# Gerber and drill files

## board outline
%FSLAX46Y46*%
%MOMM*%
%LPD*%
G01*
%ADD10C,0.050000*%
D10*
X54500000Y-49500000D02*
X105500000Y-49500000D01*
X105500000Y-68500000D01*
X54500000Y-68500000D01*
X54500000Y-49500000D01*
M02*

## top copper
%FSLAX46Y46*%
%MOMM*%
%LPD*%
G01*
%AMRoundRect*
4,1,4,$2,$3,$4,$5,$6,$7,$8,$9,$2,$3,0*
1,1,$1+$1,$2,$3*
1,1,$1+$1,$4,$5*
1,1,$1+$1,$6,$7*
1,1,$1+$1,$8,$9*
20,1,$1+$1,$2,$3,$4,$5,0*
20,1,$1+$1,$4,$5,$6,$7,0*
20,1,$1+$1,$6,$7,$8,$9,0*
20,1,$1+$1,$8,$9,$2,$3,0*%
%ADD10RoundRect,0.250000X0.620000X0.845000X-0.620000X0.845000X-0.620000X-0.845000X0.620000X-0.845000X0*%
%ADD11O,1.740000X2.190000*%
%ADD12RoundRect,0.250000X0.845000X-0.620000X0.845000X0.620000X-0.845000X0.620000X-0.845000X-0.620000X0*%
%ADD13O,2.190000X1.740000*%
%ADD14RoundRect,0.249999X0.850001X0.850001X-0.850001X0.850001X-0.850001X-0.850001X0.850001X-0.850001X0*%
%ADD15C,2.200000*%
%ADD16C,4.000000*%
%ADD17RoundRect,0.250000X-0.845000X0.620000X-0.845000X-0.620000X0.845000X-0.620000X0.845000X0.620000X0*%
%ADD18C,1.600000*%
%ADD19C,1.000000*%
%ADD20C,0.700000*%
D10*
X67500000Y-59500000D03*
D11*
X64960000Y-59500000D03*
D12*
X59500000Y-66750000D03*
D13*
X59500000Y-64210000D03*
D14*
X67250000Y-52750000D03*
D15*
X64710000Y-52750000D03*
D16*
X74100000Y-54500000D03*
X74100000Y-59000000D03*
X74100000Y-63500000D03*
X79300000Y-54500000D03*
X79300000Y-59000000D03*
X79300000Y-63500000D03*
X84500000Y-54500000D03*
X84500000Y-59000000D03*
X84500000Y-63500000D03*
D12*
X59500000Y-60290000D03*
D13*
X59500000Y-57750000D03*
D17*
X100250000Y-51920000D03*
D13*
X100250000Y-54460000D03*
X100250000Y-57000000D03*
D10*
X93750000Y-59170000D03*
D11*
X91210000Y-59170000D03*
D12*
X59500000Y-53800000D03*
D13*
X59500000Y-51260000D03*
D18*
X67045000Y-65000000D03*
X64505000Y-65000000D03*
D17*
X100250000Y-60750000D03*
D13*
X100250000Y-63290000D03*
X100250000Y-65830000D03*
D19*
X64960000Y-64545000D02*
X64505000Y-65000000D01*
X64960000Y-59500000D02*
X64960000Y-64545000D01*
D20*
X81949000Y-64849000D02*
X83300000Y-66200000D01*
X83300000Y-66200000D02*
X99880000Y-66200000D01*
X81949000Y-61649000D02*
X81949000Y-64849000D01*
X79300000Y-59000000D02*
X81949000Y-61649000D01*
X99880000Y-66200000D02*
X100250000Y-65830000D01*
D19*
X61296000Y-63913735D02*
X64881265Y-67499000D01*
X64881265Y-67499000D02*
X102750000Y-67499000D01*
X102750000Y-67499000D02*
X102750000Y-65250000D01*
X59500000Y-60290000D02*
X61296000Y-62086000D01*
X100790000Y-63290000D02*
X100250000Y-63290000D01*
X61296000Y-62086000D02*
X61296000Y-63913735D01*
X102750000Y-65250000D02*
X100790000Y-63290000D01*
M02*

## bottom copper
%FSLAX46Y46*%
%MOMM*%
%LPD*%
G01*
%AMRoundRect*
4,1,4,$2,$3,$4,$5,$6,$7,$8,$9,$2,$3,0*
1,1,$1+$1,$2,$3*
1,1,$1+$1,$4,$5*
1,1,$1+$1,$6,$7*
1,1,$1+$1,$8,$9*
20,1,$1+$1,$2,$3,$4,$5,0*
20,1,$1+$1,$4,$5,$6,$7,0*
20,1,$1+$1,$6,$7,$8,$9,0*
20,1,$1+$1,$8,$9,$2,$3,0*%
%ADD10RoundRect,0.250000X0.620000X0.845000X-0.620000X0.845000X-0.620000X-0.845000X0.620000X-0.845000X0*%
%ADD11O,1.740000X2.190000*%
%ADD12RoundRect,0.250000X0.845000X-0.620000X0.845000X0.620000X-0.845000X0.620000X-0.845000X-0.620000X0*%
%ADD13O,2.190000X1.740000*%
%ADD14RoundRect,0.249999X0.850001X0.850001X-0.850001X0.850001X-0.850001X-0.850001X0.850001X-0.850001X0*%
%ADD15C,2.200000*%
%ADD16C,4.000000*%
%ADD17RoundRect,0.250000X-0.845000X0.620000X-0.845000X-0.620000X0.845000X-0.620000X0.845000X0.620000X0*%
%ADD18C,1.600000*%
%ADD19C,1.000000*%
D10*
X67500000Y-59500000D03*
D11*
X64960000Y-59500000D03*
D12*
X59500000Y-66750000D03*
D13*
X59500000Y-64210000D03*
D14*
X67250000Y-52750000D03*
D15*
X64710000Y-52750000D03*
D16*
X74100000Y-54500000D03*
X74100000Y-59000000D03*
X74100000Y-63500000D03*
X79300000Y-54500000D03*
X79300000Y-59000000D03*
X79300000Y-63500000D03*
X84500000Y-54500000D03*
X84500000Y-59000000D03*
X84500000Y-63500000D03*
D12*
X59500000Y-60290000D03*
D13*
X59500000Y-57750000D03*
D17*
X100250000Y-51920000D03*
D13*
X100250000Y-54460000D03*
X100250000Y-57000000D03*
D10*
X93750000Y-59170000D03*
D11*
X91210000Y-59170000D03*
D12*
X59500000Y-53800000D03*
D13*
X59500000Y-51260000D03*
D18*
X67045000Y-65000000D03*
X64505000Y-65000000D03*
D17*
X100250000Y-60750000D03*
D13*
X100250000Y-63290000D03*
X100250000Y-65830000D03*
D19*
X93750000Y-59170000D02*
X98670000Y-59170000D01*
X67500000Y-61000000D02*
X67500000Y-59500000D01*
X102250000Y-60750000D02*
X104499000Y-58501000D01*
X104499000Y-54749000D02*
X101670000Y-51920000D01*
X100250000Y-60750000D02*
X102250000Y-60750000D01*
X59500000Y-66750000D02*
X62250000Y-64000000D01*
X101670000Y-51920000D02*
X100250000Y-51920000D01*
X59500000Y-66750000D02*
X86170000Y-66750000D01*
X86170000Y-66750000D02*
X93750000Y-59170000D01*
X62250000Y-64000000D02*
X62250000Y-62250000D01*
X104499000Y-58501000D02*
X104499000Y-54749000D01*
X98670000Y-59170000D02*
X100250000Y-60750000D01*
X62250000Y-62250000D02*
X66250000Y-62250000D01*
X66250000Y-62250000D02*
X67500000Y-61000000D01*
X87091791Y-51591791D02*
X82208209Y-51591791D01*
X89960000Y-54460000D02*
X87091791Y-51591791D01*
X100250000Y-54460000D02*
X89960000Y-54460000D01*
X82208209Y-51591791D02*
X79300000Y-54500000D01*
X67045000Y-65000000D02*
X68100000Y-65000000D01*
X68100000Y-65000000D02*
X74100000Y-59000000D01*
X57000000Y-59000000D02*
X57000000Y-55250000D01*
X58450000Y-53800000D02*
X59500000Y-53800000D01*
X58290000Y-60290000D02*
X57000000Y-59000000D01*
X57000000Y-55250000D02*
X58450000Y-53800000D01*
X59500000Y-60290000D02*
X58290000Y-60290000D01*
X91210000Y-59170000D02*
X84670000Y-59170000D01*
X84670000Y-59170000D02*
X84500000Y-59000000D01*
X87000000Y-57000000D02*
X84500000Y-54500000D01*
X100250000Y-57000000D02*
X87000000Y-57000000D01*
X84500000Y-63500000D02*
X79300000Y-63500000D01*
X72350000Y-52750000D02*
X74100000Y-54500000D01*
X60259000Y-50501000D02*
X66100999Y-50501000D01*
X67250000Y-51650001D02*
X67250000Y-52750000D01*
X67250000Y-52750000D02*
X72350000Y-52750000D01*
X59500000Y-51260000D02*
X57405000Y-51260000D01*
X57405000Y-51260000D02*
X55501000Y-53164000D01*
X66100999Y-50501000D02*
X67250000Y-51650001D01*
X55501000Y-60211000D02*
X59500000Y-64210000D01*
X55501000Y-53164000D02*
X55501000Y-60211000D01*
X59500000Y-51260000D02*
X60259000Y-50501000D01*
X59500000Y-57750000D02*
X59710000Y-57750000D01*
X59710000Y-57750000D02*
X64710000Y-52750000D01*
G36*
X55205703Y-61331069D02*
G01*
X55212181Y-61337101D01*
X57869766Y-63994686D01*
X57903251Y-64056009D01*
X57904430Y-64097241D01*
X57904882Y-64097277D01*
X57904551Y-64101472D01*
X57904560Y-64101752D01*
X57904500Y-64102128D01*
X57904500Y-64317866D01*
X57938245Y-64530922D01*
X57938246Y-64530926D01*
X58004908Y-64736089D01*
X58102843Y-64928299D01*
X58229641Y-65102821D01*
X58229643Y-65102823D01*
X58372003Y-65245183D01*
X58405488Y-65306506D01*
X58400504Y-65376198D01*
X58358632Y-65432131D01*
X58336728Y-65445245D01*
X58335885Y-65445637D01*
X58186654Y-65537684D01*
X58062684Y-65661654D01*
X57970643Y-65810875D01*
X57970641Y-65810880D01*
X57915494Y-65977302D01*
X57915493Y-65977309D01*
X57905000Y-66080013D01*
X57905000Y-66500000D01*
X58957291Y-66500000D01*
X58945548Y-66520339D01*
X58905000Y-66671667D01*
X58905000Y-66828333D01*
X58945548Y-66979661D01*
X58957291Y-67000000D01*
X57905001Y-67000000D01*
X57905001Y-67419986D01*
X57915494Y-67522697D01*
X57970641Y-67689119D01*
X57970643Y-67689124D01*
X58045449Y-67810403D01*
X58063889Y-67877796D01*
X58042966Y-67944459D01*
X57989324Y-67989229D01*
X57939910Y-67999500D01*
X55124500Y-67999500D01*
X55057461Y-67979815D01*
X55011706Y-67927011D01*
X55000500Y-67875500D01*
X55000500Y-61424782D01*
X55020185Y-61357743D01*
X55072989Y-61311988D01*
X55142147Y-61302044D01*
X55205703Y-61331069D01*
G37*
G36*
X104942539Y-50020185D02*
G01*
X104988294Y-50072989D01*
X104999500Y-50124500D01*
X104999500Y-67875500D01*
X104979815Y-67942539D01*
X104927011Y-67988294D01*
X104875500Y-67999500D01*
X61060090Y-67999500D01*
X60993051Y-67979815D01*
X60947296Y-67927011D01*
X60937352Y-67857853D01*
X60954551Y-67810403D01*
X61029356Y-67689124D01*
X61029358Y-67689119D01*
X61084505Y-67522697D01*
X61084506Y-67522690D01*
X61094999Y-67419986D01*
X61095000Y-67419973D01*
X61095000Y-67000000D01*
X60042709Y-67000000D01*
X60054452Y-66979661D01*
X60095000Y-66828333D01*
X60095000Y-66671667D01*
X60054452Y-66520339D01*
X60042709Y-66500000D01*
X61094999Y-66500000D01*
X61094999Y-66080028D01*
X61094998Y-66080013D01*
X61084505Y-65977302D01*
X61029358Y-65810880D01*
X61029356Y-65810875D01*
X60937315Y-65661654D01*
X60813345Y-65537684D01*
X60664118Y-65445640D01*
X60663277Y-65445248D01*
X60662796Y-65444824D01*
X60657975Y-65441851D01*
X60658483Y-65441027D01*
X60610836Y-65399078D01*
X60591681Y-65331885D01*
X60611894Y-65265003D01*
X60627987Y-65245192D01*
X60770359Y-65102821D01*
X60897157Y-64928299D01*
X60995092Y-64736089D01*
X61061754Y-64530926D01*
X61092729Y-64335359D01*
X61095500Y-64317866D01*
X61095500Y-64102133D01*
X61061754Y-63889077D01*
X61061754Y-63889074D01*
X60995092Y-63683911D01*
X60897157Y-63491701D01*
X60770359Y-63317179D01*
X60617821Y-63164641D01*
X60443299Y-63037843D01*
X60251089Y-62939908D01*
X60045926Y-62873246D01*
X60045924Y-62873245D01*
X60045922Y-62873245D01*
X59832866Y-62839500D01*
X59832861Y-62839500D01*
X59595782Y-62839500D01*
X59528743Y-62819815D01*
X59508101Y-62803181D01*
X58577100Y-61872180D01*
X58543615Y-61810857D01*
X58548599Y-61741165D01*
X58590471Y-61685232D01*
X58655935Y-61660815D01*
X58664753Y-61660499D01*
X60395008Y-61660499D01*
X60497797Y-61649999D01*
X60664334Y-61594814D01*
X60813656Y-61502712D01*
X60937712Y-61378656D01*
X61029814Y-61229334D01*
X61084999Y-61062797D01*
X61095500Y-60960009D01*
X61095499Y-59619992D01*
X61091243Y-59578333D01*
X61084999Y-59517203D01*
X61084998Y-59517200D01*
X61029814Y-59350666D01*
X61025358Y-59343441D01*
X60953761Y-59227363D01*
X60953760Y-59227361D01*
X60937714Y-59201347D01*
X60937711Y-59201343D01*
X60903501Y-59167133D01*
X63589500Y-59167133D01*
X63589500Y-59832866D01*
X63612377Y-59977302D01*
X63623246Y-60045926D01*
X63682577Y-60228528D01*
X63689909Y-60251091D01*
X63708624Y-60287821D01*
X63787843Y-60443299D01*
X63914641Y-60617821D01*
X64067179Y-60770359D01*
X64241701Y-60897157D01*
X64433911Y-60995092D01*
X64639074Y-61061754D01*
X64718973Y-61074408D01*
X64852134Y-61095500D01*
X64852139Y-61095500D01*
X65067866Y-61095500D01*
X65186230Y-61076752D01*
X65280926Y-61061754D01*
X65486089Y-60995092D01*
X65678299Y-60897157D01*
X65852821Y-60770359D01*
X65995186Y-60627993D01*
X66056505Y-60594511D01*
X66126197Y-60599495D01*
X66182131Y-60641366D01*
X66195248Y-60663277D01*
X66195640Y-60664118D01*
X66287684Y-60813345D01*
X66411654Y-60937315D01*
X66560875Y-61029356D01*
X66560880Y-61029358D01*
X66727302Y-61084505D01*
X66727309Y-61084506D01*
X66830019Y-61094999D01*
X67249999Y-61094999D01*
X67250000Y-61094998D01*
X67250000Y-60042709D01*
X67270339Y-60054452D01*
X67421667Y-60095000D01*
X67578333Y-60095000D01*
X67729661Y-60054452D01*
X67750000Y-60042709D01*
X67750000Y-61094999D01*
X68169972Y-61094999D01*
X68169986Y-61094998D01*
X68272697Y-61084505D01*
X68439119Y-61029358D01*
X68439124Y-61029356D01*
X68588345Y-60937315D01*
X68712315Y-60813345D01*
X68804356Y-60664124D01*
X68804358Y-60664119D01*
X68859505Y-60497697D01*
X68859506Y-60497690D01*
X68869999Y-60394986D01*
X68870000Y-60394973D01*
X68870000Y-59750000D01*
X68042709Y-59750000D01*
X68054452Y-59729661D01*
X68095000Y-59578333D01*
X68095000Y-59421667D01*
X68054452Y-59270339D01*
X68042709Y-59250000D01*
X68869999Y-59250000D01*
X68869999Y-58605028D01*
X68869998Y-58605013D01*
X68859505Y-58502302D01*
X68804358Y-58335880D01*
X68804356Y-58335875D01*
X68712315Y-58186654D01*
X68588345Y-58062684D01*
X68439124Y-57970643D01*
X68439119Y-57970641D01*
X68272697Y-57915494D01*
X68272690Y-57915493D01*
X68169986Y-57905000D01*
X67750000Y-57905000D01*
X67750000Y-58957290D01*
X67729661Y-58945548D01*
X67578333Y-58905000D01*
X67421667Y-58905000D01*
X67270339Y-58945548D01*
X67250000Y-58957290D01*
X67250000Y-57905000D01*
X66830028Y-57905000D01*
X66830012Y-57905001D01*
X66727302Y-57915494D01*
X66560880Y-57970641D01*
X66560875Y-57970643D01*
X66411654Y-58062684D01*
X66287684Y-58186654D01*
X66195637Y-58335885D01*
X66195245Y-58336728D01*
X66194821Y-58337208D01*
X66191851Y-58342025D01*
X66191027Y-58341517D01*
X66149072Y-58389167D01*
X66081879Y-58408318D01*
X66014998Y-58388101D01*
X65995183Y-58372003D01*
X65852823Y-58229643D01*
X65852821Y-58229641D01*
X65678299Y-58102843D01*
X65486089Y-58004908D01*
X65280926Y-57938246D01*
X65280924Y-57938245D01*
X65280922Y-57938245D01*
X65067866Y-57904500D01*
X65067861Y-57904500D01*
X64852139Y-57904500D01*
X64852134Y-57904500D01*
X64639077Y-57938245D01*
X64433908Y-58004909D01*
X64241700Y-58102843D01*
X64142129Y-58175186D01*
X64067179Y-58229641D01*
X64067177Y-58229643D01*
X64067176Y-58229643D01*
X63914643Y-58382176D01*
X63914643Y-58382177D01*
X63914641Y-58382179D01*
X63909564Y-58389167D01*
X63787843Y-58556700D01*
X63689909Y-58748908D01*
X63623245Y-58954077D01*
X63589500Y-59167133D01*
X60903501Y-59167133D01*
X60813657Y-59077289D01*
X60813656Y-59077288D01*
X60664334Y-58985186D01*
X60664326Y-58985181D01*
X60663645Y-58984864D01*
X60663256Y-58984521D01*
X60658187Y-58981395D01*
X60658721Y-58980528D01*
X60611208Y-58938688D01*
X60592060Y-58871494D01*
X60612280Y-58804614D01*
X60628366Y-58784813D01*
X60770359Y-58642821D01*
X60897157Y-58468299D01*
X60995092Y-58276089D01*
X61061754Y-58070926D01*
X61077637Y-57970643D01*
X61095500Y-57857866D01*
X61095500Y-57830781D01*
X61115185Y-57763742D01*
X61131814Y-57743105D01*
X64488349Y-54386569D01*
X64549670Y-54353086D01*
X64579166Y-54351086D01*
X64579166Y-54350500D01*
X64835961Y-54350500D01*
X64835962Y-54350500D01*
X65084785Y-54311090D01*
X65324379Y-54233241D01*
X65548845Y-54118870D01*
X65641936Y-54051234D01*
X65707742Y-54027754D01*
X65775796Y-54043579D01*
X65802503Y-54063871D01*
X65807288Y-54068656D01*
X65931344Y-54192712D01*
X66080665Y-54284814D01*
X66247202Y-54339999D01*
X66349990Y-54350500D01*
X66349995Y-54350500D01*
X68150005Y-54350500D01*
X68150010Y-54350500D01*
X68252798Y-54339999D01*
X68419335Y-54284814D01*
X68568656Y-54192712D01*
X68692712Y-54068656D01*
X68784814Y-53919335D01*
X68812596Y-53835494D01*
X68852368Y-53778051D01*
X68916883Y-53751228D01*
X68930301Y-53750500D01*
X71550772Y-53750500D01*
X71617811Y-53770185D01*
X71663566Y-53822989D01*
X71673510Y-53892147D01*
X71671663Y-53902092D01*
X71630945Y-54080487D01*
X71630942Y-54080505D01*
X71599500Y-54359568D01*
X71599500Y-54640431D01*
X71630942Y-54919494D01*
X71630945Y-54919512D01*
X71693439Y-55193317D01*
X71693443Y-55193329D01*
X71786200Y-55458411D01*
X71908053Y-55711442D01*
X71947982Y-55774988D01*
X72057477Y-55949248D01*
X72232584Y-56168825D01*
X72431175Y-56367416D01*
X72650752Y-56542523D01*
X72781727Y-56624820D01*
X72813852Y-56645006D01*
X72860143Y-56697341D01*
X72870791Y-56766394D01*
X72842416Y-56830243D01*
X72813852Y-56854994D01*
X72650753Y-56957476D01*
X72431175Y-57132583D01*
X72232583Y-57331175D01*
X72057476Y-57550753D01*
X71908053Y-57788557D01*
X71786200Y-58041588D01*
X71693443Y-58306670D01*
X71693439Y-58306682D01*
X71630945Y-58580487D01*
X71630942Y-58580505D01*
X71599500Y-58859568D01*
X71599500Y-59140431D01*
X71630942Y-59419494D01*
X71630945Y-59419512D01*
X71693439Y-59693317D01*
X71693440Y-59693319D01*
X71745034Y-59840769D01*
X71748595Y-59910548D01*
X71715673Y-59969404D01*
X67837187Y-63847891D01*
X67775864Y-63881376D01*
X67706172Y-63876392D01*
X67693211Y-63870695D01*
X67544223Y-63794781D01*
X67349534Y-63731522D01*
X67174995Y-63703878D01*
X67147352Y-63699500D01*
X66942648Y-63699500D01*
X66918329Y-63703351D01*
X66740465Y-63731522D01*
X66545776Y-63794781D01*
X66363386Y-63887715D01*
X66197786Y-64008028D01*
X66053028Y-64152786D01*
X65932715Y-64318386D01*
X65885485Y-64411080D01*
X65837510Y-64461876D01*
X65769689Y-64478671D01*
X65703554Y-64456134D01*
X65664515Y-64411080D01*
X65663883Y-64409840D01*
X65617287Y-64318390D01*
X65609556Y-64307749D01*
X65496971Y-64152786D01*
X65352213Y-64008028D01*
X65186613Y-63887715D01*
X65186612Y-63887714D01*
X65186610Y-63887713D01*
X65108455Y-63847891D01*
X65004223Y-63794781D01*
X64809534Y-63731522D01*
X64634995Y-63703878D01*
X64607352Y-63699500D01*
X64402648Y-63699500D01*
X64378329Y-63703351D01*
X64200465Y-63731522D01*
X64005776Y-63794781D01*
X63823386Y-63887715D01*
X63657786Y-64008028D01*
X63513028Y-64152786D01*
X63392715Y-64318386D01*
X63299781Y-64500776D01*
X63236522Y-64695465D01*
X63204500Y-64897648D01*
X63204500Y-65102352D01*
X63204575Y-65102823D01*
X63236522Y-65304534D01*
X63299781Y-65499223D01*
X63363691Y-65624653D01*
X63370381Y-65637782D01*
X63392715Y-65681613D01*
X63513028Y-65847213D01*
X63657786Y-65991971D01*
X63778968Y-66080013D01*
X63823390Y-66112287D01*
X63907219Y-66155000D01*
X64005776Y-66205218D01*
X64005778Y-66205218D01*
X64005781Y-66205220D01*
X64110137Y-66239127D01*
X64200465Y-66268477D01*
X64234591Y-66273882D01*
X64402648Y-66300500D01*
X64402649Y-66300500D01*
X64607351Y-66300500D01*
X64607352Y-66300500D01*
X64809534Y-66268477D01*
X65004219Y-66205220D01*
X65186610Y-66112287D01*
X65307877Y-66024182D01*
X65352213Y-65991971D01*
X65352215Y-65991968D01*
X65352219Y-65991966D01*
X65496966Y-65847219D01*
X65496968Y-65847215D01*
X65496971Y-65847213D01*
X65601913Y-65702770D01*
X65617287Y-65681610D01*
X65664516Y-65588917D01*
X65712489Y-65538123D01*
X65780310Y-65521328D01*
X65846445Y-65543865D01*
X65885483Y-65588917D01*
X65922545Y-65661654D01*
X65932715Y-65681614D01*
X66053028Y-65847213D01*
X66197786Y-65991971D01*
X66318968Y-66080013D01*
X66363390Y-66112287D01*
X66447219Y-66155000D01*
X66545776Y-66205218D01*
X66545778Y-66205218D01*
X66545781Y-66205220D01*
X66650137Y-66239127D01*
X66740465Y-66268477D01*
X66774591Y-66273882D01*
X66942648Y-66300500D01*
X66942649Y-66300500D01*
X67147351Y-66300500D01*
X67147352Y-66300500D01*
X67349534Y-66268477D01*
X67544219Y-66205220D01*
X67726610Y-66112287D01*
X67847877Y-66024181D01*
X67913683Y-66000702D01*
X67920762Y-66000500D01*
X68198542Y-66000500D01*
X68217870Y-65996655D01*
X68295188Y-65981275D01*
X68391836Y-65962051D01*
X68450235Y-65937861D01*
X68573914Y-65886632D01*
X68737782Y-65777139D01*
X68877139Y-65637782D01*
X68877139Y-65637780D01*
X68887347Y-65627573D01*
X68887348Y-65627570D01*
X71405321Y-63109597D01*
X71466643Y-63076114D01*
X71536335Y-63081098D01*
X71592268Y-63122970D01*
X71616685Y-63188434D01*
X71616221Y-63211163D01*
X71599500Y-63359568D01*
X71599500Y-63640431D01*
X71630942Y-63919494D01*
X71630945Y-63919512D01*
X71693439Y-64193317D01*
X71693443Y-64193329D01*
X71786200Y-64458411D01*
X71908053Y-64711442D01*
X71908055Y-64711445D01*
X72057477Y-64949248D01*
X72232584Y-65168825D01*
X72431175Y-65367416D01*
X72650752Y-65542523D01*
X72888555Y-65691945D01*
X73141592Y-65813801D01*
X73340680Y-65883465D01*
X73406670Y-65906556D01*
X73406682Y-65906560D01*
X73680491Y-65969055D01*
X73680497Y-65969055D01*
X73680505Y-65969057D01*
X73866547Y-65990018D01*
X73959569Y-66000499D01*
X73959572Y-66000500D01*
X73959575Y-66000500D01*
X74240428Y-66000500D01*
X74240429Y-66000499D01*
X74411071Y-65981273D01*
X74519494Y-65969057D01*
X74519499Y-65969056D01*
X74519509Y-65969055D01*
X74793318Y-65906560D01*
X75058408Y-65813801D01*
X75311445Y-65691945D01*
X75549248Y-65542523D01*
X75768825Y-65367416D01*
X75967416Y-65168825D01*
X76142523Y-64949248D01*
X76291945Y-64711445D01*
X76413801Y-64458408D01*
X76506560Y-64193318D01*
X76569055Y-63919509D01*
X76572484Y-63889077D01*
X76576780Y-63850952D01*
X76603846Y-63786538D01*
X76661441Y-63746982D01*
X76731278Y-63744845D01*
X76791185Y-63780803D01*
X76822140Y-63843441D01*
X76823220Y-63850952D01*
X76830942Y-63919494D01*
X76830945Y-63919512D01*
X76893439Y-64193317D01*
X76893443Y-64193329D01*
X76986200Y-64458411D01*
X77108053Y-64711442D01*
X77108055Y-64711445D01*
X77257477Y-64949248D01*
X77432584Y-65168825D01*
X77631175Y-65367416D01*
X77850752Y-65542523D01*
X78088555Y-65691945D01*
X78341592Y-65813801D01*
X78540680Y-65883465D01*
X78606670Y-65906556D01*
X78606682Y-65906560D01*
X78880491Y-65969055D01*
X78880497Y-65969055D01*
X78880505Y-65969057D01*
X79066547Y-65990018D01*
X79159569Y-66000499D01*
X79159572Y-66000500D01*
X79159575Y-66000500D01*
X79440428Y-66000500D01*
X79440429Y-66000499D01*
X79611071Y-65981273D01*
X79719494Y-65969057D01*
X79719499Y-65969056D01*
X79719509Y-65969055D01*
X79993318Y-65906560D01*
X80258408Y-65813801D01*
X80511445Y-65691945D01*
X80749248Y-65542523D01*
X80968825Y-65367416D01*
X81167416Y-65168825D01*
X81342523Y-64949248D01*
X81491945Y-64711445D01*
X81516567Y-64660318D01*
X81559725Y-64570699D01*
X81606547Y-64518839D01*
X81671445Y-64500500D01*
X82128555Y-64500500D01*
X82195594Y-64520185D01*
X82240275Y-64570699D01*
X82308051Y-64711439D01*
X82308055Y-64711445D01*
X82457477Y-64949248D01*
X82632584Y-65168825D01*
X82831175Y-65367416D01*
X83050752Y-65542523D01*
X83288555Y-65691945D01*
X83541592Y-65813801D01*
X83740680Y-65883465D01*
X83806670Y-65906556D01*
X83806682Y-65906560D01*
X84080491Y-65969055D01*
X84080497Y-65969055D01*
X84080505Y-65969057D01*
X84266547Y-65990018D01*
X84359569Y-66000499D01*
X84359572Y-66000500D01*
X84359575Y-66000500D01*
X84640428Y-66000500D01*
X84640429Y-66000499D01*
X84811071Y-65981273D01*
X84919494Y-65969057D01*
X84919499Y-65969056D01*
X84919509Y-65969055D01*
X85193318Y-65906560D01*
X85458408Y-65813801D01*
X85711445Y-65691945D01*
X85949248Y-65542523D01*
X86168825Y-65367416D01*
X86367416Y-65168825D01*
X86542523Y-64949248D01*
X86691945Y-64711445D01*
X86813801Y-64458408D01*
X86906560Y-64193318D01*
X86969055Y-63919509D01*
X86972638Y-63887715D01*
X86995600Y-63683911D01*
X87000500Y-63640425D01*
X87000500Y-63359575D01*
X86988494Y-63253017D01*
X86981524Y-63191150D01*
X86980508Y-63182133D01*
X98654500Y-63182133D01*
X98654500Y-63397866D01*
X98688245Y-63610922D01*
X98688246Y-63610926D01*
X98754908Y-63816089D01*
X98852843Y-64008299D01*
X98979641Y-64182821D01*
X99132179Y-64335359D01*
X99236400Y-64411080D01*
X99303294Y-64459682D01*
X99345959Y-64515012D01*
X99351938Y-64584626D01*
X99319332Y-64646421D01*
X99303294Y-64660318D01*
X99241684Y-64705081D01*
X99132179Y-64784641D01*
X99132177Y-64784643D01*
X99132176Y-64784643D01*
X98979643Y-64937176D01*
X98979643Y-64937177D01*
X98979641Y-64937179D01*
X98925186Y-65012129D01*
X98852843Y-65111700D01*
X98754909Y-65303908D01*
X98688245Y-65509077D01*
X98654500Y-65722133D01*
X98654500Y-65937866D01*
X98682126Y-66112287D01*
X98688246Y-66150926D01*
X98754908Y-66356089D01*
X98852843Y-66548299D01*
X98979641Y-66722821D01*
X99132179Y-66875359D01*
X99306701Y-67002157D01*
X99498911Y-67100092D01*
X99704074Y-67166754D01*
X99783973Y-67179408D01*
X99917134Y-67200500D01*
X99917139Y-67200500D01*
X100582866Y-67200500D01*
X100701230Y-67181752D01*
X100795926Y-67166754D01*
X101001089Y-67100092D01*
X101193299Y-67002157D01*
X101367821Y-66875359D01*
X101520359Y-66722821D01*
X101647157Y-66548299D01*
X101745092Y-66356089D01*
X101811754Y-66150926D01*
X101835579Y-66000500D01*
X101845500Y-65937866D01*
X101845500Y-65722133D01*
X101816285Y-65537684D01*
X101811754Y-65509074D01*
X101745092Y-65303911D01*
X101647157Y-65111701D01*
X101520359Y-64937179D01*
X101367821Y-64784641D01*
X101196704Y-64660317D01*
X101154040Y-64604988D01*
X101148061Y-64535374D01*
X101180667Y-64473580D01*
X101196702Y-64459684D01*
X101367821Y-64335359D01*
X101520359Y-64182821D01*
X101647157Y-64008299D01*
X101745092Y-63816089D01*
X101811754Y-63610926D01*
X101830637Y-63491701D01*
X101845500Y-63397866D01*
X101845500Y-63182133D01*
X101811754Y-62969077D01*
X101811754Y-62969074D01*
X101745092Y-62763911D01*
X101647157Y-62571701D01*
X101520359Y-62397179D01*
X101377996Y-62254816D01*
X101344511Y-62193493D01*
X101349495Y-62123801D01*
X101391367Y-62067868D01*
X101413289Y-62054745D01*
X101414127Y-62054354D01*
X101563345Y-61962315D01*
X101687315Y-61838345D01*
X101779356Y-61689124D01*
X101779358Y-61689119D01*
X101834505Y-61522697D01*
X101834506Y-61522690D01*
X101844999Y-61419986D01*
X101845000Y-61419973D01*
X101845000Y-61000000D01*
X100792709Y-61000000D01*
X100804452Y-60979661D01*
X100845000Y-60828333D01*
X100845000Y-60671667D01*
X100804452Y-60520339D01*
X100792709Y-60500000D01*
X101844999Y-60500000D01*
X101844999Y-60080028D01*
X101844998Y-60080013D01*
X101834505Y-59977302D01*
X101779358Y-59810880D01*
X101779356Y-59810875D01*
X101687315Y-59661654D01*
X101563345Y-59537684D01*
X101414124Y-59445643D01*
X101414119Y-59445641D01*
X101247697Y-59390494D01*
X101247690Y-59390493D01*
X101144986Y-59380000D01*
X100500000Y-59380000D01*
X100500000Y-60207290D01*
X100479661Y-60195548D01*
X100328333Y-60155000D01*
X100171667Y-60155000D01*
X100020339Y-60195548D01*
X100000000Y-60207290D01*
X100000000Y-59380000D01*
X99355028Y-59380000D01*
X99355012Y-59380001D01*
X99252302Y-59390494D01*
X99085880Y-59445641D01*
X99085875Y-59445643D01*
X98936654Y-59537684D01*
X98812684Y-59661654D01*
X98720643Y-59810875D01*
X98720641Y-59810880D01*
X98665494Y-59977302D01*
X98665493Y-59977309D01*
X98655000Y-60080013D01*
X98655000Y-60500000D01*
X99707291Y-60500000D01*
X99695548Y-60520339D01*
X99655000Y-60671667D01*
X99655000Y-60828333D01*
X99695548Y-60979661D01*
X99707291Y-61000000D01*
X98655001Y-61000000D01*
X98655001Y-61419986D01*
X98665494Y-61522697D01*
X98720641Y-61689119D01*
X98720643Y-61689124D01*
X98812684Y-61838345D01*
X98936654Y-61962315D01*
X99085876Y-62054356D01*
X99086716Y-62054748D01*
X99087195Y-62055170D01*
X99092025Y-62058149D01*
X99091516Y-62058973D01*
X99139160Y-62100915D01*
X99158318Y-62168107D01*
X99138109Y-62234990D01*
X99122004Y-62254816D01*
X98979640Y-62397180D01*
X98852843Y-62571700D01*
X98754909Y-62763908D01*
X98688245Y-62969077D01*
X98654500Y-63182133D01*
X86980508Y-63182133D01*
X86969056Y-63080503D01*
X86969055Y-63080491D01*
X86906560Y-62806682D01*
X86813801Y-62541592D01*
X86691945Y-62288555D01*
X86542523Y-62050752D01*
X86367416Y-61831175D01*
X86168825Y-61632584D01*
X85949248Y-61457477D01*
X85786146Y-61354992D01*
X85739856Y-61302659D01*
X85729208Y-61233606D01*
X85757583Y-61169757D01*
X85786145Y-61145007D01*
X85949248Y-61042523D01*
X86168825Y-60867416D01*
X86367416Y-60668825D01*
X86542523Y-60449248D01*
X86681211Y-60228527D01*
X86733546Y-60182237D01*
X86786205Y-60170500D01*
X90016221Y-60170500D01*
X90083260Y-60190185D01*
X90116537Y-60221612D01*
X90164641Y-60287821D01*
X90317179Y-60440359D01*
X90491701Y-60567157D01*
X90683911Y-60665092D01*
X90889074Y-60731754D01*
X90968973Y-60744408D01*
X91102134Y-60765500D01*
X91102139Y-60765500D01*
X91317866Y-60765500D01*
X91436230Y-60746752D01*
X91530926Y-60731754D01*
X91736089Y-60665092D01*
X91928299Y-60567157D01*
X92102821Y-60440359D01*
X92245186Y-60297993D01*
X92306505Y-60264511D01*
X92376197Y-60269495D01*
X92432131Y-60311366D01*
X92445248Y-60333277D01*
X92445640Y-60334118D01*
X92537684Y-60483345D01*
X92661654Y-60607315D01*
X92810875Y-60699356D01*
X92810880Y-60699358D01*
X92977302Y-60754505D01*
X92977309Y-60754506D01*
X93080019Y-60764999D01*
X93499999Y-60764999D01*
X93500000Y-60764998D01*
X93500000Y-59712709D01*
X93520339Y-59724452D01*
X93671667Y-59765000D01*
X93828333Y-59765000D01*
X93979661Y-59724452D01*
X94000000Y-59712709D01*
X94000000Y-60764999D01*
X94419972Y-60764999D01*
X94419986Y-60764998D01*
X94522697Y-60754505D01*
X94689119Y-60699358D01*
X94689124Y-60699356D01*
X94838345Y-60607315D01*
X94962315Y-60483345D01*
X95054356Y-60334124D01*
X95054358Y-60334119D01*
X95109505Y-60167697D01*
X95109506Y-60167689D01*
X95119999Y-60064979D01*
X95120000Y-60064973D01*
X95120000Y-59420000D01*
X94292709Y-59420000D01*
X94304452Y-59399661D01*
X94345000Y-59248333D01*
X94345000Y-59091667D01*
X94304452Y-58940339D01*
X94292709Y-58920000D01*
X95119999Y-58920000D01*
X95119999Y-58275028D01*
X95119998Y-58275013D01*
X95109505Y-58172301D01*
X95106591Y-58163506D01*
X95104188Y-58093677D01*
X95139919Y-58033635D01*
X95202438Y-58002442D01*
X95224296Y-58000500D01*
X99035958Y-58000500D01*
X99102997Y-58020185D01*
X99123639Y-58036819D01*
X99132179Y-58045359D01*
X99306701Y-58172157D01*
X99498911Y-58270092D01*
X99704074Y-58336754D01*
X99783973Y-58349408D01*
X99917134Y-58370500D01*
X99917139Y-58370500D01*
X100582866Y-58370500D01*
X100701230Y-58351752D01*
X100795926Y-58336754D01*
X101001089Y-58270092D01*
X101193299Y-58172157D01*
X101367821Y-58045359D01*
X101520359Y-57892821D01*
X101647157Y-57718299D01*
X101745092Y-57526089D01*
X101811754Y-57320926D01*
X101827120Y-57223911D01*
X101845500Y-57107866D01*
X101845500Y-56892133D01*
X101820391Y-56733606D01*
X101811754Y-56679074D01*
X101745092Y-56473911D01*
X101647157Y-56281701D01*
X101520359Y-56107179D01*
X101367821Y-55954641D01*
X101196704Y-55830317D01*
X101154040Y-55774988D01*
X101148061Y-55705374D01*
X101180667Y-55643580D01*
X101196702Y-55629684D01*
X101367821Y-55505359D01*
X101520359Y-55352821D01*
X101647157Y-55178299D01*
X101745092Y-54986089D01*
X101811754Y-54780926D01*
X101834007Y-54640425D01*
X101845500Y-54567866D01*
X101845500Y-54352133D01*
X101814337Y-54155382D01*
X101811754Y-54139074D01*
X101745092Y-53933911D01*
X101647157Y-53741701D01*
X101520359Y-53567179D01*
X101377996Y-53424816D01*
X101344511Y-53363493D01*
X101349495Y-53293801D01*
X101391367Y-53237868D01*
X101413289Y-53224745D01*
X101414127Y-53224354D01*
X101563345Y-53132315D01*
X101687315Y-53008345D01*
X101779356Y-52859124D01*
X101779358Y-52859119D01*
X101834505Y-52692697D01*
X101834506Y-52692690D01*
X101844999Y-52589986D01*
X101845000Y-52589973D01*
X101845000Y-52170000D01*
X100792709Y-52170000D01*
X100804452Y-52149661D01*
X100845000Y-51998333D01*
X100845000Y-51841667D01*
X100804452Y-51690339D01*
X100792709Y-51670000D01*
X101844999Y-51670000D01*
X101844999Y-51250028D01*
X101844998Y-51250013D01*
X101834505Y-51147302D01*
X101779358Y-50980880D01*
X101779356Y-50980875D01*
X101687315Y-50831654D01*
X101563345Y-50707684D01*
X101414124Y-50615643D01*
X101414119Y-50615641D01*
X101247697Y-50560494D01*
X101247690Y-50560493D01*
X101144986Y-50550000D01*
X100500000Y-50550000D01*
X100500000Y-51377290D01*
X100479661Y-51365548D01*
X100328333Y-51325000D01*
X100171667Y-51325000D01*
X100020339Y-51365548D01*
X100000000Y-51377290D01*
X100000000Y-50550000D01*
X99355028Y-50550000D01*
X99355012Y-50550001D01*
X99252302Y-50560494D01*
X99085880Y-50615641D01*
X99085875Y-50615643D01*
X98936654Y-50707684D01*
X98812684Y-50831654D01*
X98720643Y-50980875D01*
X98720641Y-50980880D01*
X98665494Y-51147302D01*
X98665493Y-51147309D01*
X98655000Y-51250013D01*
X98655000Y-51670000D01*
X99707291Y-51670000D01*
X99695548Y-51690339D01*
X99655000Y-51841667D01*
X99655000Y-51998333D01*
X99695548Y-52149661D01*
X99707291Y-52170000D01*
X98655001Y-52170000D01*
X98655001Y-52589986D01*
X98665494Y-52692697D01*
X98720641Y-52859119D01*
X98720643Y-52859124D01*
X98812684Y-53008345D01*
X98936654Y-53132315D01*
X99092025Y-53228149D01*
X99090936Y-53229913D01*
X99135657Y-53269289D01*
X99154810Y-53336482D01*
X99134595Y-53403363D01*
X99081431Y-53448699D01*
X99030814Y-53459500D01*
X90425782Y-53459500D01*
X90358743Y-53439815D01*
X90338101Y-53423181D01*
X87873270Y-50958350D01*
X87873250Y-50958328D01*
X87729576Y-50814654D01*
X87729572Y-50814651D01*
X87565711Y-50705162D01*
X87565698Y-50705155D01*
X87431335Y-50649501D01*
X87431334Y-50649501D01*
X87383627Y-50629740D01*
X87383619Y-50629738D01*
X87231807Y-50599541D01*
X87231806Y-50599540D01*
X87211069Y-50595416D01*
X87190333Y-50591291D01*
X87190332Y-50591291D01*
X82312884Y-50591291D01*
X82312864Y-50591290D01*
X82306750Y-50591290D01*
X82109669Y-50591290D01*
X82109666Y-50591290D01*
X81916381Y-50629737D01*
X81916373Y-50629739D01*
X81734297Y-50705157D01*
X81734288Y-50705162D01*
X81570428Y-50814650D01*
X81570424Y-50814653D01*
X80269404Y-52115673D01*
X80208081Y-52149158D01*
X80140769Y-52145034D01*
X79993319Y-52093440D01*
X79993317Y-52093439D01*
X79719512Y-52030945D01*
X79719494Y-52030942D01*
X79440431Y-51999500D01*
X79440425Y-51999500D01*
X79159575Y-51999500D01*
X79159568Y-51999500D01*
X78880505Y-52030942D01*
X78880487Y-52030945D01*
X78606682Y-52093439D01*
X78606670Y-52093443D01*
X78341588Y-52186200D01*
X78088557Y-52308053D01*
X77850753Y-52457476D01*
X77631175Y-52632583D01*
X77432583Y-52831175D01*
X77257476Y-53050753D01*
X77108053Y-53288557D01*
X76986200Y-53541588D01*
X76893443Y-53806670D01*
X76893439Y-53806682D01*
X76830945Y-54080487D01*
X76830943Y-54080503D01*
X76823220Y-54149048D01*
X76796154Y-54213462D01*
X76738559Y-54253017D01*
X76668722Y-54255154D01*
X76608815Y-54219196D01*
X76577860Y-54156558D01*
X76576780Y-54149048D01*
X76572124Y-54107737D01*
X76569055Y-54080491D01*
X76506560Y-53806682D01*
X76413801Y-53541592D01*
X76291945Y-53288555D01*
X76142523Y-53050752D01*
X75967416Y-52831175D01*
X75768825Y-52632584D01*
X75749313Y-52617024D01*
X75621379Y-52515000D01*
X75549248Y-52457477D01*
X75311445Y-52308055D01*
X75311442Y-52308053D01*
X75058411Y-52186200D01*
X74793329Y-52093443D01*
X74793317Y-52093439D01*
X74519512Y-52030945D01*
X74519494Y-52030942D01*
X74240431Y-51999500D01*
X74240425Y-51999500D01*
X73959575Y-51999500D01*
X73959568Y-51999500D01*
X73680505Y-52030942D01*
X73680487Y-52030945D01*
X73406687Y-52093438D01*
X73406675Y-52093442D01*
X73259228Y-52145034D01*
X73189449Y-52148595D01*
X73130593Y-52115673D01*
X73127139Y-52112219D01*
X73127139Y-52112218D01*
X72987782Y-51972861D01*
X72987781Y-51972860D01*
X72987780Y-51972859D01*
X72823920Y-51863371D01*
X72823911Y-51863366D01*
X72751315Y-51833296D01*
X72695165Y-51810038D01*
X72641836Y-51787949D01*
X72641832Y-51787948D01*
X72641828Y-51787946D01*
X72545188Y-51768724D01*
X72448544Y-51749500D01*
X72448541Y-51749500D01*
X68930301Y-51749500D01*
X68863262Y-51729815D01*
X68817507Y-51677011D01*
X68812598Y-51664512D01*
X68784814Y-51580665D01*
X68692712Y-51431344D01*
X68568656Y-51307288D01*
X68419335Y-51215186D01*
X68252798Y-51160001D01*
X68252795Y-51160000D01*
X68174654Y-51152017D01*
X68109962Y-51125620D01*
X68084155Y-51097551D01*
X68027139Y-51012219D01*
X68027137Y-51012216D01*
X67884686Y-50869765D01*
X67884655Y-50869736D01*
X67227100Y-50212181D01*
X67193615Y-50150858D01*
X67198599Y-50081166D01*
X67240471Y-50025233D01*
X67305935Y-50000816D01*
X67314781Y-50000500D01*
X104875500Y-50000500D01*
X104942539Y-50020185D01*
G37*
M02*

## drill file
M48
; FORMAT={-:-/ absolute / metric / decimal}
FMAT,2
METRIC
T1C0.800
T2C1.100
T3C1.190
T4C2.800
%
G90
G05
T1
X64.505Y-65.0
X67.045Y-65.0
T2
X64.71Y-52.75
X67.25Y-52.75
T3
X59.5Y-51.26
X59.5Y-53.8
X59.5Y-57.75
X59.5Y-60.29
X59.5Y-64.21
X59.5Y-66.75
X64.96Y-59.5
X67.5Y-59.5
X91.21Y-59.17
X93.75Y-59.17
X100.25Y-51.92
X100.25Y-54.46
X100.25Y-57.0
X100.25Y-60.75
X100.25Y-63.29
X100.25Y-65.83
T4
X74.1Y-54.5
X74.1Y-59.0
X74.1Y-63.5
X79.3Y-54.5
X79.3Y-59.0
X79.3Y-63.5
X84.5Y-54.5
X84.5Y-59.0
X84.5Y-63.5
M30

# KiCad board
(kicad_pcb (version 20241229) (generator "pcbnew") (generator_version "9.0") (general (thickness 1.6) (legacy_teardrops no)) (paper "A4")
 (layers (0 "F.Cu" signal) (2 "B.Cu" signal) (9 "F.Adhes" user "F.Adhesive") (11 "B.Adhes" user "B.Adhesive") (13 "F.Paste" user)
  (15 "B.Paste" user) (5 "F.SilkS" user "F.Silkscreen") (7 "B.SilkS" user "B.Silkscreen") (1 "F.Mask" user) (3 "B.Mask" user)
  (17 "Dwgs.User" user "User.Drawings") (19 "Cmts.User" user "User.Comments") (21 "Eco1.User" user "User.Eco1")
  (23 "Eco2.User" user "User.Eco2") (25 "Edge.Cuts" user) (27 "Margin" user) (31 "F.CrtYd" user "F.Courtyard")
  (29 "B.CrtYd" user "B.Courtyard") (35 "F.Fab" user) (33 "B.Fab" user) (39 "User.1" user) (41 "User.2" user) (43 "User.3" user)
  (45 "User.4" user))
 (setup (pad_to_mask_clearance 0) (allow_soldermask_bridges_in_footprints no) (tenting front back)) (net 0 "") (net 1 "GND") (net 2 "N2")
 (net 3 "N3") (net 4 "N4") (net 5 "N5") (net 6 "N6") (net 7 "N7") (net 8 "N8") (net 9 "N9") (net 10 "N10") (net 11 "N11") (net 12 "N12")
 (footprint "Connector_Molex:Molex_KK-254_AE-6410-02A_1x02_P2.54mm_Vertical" (layer "F.Cu") (at 67.5 59.5 180)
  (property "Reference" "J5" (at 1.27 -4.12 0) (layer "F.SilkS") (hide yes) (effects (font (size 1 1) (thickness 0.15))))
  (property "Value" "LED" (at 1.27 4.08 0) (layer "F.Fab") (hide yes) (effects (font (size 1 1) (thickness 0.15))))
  (pad "1" thru_hole roundrect (at 0 0 180) (size 1.74 2.19) (drill 1.19) (layers "*.Cu" "*.Mask") (remove_unused_layers no)
   (roundrect_rratio 0.143678) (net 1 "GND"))
  (pad "2" thru_hole oval (at 2.54 0 180) (size 1.74 2.19) (drill 1.19) (layers "*.Cu" "*.Mask") (remove_unused_layers no) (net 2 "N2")))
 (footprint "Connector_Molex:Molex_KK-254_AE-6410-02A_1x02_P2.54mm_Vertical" (layer "F.Cu") (at 59.5 66.75 90)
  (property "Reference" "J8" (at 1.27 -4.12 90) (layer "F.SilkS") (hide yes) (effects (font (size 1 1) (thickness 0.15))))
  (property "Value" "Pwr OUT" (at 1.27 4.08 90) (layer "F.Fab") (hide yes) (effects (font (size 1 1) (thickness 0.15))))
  (pad "1" thru_hole roundrect (at 0 0 90) (size 1.74 2.19) (drill 1.19) (layers "*.Cu" "*.Mask") (remove_unused_layers no)
   (roundrect_rratio 0.143678) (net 1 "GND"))
  (pad "2" thru_hole oval (at 2.54 0 90) (size 1.74 2.19) (drill 1.19) (layers "*.Cu" "*.Mask") (remove_unused_layers no) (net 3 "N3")))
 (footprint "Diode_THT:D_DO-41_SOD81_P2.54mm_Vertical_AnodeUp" (layer "F.Cu") (at 67.25 52.75 180)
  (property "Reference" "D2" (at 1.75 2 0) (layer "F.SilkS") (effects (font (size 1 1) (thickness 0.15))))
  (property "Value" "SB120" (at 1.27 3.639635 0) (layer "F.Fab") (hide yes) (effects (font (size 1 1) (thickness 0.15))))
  (pad "1" thru_hole roundrect (at 0 0 180) (size 2.2 2.2) (drill 1.1) (layers "*.Cu" "*.Mask") (remove_unused_layers no)
   (roundrect_rratio 0.113636) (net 3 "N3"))
  (pad "2" thru_hole circle (at 2.54 0 180) (size 2.2 2.2) (drill 1.1) (layers "*.Cu" "*.Mask") (remove_unused_layers no) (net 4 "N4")))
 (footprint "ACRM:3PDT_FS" (layer "F.Cu") (at 77.1 58)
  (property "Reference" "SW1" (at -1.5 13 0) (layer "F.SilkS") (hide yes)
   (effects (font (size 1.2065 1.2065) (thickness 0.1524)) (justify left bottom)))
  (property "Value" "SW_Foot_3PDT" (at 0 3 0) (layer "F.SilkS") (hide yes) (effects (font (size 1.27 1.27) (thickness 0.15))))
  (pad "A1" thru_hole circle (at -3 -3.5 180) (size 4 4) (drill 2.8) (layers "*.Cu" "*.Mask") (remove_unused_layers no) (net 3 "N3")
   (solder_mask_margin 0.1016))
  (pad "A2" thru_hole circle (at -3 1 180) (size 4 4) (drill 2.8) (layers "*.Cu" "*.Mask") (remove_unused_layers no) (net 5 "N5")
   (solder_mask_margin 0.1016))
  (pad "A3" thru_hole circle (at -3 5.5 180) (size 4 4) (drill 2.8) (layers "*.Cu" "*.Mask") (remove_unused_layers no) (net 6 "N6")
   (solder_mask_margin 0.1016))
  (pad "B1" thru_hole circle (at 2.2 -3.5 180) (size 4 4) (drill 2.8) (layers "*.Cu" "*.Mask") (remove_unused_layers no) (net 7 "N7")
   (solder_mask_margin 0.1016))
  (pad "B2" thru_hole circle (at 2.2 1 180) (size 4 4) (drill 2.8) (layers "*.Cu" "*.Mask") (remove_unused_layers no) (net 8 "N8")
   (solder_mask_margin 0.1016))
  (pad "B3" thru_hole circle (at 2.2 5.5 180) (size 4 4) (drill 2.8) (layers "*.Cu" "*.Mask") (remove_unused_layers no) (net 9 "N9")
   (solder_mask_margin 0.1016))
  (pad "C1" thru_hole circle (at 7.4 -3.5 180) (size 4 4) (drill 2.8) (layers "*.Cu" "*.Mask") (remove_unused_layers no) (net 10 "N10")
   (solder_mask_margin 0.1016))
  (pad "C2" thru_hole circle (at 7.4 1 180) (size 4 4) (drill 2.8) (layers "*.Cu" "*.Mask") (remove_unused_layers no) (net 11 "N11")
   (solder_mask_margin 0.1016))
  (pad "C3" thru_hole circle (at 7.4 5.5 180) (size 4 4) (drill 2.8) (layers "*.Cu" "*.Mask") (remove_unused_layers no) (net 9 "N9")
   (solder_mask_margin 0.1016)))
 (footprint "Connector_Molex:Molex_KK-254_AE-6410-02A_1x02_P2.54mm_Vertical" (layer "F.Cu") (at 59.5 60.29 90)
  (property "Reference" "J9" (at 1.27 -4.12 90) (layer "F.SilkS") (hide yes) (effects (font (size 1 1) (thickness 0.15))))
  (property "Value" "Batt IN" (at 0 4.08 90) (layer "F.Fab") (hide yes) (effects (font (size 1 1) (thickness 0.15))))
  (pad "1" thru_hole roundrect (at 0 0 90) (size 1.74 2.19) (drill 1.19) (layers "*.Cu" "*.Mask") (remove_unused_layers no)
   (roundrect_rratio 0.143678) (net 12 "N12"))
  (pad "2" thru_hole oval (at 2.54 0 90) (size 1.74 2.19) (drill 1.19) (layers "*.Cu" "*.Mask") (remove_unused_layers no) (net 4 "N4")))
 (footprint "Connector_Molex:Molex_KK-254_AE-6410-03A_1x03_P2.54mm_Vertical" (layer "F.Cu") (at 100.25 51.92 -90)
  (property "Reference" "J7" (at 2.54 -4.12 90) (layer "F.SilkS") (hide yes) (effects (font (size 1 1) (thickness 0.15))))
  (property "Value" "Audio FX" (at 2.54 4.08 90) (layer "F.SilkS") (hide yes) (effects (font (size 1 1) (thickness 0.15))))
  (pad "1" thru_hole roundrect (at 0 0 270) (size 1.74 2.19) (drill 1.19) (layers "*.Cu" "*.Mask") (remove_unused_layers no)
   (roundrect_rratio 0.143678) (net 1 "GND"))
  (pad "2" thru_hole oval (at 2.54 0 270) (size 1.74 2.19) (drill 1.19) (layers "*.Cu" "*.Mask") (remove_unused_layers no) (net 7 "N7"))
  (pad "3" thru_hole oval (at 5.08 0 270) (size 1.74 2.19) (drill 1.19) (layers "*.Cu" "*.Mask") (remove_unused_layers no) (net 10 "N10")))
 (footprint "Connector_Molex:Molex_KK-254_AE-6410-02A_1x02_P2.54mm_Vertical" (layer "F.Cu") (at 93.75 59.17 180)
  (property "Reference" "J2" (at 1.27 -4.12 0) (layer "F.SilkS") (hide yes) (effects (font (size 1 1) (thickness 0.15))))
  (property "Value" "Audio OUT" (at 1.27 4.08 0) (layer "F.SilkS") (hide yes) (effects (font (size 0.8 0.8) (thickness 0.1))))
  (pad "1" thru_hole roundrect (at 0 0 180) (size 1.74 2.19) (drill 1.19) (layers "*.Cu" "*.Mask") (remove_unused_layers no)
   (roundrect_rratio 0.143678) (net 1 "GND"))
  (pad "2" thru_hole oval (at 2.54 0 180) (size 1.74 2.19) (drill 1.19) (layers "*.Cu" "*.Mask") (remove_unused_layers no) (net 11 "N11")))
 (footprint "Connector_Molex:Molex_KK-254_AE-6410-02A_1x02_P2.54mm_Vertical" (layer "F.Cu") (at 59.5 53.8 90)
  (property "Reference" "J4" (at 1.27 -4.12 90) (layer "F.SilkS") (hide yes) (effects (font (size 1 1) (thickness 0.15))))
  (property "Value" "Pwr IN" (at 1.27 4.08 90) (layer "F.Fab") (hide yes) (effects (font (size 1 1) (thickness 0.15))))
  (pad "1" thru_hole roundrect (at 0 0 90) (size 1.74 2.19) (drill 1.19) (layers "*.Cu" "*.Mask") (remove_unused_layers no)
   (roundrect_rratio 0.143678) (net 12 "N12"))
  (pad "2" thru_hole oval (at 2.54 0 90) (size 1.74 2.19) (drill 1.19) (layers "*.Cu" "*.Mask") (remove_unused_layers no) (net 3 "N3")))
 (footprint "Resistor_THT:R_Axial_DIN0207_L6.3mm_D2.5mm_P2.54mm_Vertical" (layer "F.Cu") (at 67.045 65 180)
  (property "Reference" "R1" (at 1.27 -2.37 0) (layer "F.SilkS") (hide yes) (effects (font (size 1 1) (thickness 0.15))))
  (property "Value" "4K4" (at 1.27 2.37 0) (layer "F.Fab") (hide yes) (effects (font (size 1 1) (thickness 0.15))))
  (pad "1" thru_hole circle (at 0 0 180) (size 1.6 1.6) (drill 0.8) (layers "*.Cu" "*.Mask") (remove_unused_layers no) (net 5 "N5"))
  (pad "2" thru_hole circle (at 2.54 0 180) (size 1.6 1.6) (drill 0.8) (layers "*.Cu" "*.Mask") (remove_unused_layers no) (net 2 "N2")))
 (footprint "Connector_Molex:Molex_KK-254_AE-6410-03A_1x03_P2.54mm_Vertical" (layer "F.Cu") (at 100.25 60.75 -90)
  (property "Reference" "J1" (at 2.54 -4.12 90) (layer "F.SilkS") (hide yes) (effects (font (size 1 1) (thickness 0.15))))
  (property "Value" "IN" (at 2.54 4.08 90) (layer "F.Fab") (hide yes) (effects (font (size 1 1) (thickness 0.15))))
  (pad "1" thru_hole roundrect (at 0 0 270) (size 1.74 2.19) (drill 1.19) (layers "*.Cu" "*.Mask") (remove_unused_layers no)
   (roundrect_rratio 0.143678) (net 1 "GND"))
  (pad "2" thru_hole oval (at 2.54 0 270) (size 1.74 2.19) (drill 1.19) (layers "*.Cu" "*.Mask") (remove_unused_layers no) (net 12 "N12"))
  (pad "3" thru_hole oval (at 5.08 0 270) (size 1.74 2.19) (drill 1.19) (layers "*.Cu" "*.Mask") (remove_unused_layers no) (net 8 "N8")))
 (gr_rect (start 54.5 49.5) (end 105.5 68.5) (stroke (width 0.05) (type default)) (fill no) (layer "Edge.Cuts"))
 (segment (start 93.75 59.17) (end 98.67 59.17) (width 1) (layer "B.Cu") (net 1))
 (segment (start 67.5 61) (end 67.5 59.5) (width 1) (layer "B.Cu") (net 1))
 (segment (start 102.25 60.75) (end 104.499 58.501) (width 1) (layer "B.Cu") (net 1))
 (segment (start 104.499 54.749) (end 101.67 51.92) (width 1) (layer "B.Cu") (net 1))
 (segment (start 100.25 60.75) (end 102.25 60.75) (width 1) (layer "B.Cu") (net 1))
 (segment (start 59.5 66.75) (end 62.25 64) (width 1) (layer "B.Cu") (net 1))
 (segment (start 101.67 51.92) (end 100.25 51.92) (width 1) (layer "B.Cu") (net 1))
 (segment (start 59.5 66.75) (end 86.17 66.75) (width 1) (layer "B.Cu") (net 1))
 (segment (start 86.17 66.75) (end 93.75 59.17) (width 1) (layer "B.Cu") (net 1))
 (segment (start 62.25 64) (end 62.25 62.25) (width 1) (layer "B.Cu") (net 1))
 (segment (start 104.499 58.501) (end 104.499 54.749) (width 1) (layer "B.Cu") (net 1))
 (segment (start 98.67 59.17) (end 100.25 60.75) (width 1) (layer "B.Cu") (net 1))
 (segment (start 62.25 62.25) (end 66.25 62.25) (width 1) (layer "B.Cu") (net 1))
 (segment (start 66.25 62.25) (end 67.5 61) (width 1) (layer "B.Cu") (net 1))
 (segment (start 64.96 64.545) (end 64.505 65) (width 1) (layer "F.Cu") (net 2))
 (segment (start 64.96 59.5) (end 64.96 64.545) (width 1) (layer "F.Cu") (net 2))
 (segment (start 87.091791 51.591791) (end 82.208209 51.591791) (width 1) (layer "B.Cu") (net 7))
 (segment (start 89.96 54.46) (end 87.091791 51.591791) (width 1) (layer "B.Cu") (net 7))
 (segment (start 100.25 54.46) (end 89.96 54.46) (width 1) (layer "B.Cu") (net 7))
 (segment (start 82.208209 51.591791) (end 79.3 54.5) (width 1) (layer "B.Cu") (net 7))
 (segment (start 67.045 65) (end 68.1 65) (width 1) (layer "B.Cu") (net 5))
 (segment (start 68.1 65) (end 74.1 59) (width 1) (layer "B.Cu") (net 5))
 (segment (start 81.949 64.849) (end 83.3 66.2) (width 0.7) (layer "F.Cu") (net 8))
 (segment (start 83.3 66.2) (end 99.88 66.2) (width 0.7) (layer "F.Cu") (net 8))
 (segment (start 81.949 61.649) (end 81.949 64.849) (width 0.7) (layer "F.Cu") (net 8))
 (segment (start 79.3 59) (end 81.949 61.649) (width 0.7) (layer "F.Cu") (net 8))
 (segment (start 99.88 66.2) (end 100.25 65.83) (width 0.7) (layer "F.Cu") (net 8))
 (segment (start 61.296 63.913735) (end 64.881265 67.499) (width 1) (layer "F.Cu") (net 12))
 (segment (start 64.881265 67.499) (end 102.75 67.499) (width 1) (layer "F.Cu") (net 12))
 (segment (start 102.75 67.499) (end 102.75 65.25) (width 1) (layer "F.Cu") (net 12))
 (segment (start 59.5 60.29) (end 61.296 62.086) (width 1) (layer "F.Cu") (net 12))
 (segment (start 100.79 63.29) (end 100.25 63.29) (width 1) (layer "F.Cu") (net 12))
 (segment (start 61.296 62.086) (end 61.296 63.913735) (width 1) (layer "F.Cu") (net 12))
 (segment (start 102.75 65.25) (end 100.79 63.29) (width 1) (layer "F.Cu") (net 12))
 (segment (start 57 59) (end 57 55.25) (width 1) (layer "B.Cu") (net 12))
 (segment (start 58.45 53.8) (end 59.5 53.8) (width 1) (layer "B.Cu") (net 12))
 (segment (start 58.29 60.29) (end 57 59) (width 1) (layer "B.Cu") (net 12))
 (segment (start 57 55.25) (end 58.45 53.8) (width 1) (layer "B.Cu") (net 12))
 (segment (start 59.5 60.29) (end 58.29 60.29) (width 1) (layer "B.Cu") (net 12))
 (segment (start 91.21 59.17) (end 84.67 59.17) (width 1) (layer "B.Cu") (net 11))
 (segment (start 84.67 59.17) (end 84.5 59) (width 1) (layer "B.Cu") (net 11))
 (segment (start 87 57) (end 84.5 54.5) (width 1) (layer "B.Cu") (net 10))
 (segment (start 100.25 57) (end 87 57) (width 1) (layer "B.Cu") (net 10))
 (segment (start 84.5 63.5) (end 79.3 63.5) (width 1) (layer "B.Cu") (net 9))
 (segment (start 72.35 52.75) (end 74.1 54.5) (width 1) (layer "B.Cu") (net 3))
 (segment (start 60.259 50.501) (end 66.100999 50.501) (width 1) (layer "B.Cu") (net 3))
 (segment (start 67.25 51.650001) (end 67.25 52.75) (width 1) (layer "B.Cu") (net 3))
 (segment (start 67.25 52.75) (end 72.35 52.75) (width 1) (layer "B.Cu") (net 3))
 (segment (start 59.5 51.26) (end 57.405 51.26) (width 1) (layer "B.Cu") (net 3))
 (segment (start 57.405 51.26) (end 55.501 53.164) (width 1) (layer "B.Cu") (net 3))
 (segment (start 66.100999 50.501) (end 67.25 51.650001) (width 1) (layer "B.Cu") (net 3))
 (segment (start 55.501 60.211) (end 59.5 64.21) (width 1) (layer "B.Cu") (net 3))
 (segment (start 55.501 53.164) (end 55.501 60.211) (width 1) (layer "B.Cu") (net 3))
 (segment (start 59.5 51.26) (end 60.259 50.501) (width 1) (layer "B.Cu") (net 3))
 (segment (start 59.5 57.75) (end 59.71 57.75) (width 1) (layer "B.Cu") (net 4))
 (segment (start 59.71 57.75) (end 64.71 52.75) (width 1) (layer "B.Cu") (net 4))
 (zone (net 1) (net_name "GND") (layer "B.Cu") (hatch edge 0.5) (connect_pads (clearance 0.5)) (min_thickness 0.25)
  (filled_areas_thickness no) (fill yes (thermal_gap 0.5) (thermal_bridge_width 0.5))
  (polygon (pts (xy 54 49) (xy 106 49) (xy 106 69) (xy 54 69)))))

